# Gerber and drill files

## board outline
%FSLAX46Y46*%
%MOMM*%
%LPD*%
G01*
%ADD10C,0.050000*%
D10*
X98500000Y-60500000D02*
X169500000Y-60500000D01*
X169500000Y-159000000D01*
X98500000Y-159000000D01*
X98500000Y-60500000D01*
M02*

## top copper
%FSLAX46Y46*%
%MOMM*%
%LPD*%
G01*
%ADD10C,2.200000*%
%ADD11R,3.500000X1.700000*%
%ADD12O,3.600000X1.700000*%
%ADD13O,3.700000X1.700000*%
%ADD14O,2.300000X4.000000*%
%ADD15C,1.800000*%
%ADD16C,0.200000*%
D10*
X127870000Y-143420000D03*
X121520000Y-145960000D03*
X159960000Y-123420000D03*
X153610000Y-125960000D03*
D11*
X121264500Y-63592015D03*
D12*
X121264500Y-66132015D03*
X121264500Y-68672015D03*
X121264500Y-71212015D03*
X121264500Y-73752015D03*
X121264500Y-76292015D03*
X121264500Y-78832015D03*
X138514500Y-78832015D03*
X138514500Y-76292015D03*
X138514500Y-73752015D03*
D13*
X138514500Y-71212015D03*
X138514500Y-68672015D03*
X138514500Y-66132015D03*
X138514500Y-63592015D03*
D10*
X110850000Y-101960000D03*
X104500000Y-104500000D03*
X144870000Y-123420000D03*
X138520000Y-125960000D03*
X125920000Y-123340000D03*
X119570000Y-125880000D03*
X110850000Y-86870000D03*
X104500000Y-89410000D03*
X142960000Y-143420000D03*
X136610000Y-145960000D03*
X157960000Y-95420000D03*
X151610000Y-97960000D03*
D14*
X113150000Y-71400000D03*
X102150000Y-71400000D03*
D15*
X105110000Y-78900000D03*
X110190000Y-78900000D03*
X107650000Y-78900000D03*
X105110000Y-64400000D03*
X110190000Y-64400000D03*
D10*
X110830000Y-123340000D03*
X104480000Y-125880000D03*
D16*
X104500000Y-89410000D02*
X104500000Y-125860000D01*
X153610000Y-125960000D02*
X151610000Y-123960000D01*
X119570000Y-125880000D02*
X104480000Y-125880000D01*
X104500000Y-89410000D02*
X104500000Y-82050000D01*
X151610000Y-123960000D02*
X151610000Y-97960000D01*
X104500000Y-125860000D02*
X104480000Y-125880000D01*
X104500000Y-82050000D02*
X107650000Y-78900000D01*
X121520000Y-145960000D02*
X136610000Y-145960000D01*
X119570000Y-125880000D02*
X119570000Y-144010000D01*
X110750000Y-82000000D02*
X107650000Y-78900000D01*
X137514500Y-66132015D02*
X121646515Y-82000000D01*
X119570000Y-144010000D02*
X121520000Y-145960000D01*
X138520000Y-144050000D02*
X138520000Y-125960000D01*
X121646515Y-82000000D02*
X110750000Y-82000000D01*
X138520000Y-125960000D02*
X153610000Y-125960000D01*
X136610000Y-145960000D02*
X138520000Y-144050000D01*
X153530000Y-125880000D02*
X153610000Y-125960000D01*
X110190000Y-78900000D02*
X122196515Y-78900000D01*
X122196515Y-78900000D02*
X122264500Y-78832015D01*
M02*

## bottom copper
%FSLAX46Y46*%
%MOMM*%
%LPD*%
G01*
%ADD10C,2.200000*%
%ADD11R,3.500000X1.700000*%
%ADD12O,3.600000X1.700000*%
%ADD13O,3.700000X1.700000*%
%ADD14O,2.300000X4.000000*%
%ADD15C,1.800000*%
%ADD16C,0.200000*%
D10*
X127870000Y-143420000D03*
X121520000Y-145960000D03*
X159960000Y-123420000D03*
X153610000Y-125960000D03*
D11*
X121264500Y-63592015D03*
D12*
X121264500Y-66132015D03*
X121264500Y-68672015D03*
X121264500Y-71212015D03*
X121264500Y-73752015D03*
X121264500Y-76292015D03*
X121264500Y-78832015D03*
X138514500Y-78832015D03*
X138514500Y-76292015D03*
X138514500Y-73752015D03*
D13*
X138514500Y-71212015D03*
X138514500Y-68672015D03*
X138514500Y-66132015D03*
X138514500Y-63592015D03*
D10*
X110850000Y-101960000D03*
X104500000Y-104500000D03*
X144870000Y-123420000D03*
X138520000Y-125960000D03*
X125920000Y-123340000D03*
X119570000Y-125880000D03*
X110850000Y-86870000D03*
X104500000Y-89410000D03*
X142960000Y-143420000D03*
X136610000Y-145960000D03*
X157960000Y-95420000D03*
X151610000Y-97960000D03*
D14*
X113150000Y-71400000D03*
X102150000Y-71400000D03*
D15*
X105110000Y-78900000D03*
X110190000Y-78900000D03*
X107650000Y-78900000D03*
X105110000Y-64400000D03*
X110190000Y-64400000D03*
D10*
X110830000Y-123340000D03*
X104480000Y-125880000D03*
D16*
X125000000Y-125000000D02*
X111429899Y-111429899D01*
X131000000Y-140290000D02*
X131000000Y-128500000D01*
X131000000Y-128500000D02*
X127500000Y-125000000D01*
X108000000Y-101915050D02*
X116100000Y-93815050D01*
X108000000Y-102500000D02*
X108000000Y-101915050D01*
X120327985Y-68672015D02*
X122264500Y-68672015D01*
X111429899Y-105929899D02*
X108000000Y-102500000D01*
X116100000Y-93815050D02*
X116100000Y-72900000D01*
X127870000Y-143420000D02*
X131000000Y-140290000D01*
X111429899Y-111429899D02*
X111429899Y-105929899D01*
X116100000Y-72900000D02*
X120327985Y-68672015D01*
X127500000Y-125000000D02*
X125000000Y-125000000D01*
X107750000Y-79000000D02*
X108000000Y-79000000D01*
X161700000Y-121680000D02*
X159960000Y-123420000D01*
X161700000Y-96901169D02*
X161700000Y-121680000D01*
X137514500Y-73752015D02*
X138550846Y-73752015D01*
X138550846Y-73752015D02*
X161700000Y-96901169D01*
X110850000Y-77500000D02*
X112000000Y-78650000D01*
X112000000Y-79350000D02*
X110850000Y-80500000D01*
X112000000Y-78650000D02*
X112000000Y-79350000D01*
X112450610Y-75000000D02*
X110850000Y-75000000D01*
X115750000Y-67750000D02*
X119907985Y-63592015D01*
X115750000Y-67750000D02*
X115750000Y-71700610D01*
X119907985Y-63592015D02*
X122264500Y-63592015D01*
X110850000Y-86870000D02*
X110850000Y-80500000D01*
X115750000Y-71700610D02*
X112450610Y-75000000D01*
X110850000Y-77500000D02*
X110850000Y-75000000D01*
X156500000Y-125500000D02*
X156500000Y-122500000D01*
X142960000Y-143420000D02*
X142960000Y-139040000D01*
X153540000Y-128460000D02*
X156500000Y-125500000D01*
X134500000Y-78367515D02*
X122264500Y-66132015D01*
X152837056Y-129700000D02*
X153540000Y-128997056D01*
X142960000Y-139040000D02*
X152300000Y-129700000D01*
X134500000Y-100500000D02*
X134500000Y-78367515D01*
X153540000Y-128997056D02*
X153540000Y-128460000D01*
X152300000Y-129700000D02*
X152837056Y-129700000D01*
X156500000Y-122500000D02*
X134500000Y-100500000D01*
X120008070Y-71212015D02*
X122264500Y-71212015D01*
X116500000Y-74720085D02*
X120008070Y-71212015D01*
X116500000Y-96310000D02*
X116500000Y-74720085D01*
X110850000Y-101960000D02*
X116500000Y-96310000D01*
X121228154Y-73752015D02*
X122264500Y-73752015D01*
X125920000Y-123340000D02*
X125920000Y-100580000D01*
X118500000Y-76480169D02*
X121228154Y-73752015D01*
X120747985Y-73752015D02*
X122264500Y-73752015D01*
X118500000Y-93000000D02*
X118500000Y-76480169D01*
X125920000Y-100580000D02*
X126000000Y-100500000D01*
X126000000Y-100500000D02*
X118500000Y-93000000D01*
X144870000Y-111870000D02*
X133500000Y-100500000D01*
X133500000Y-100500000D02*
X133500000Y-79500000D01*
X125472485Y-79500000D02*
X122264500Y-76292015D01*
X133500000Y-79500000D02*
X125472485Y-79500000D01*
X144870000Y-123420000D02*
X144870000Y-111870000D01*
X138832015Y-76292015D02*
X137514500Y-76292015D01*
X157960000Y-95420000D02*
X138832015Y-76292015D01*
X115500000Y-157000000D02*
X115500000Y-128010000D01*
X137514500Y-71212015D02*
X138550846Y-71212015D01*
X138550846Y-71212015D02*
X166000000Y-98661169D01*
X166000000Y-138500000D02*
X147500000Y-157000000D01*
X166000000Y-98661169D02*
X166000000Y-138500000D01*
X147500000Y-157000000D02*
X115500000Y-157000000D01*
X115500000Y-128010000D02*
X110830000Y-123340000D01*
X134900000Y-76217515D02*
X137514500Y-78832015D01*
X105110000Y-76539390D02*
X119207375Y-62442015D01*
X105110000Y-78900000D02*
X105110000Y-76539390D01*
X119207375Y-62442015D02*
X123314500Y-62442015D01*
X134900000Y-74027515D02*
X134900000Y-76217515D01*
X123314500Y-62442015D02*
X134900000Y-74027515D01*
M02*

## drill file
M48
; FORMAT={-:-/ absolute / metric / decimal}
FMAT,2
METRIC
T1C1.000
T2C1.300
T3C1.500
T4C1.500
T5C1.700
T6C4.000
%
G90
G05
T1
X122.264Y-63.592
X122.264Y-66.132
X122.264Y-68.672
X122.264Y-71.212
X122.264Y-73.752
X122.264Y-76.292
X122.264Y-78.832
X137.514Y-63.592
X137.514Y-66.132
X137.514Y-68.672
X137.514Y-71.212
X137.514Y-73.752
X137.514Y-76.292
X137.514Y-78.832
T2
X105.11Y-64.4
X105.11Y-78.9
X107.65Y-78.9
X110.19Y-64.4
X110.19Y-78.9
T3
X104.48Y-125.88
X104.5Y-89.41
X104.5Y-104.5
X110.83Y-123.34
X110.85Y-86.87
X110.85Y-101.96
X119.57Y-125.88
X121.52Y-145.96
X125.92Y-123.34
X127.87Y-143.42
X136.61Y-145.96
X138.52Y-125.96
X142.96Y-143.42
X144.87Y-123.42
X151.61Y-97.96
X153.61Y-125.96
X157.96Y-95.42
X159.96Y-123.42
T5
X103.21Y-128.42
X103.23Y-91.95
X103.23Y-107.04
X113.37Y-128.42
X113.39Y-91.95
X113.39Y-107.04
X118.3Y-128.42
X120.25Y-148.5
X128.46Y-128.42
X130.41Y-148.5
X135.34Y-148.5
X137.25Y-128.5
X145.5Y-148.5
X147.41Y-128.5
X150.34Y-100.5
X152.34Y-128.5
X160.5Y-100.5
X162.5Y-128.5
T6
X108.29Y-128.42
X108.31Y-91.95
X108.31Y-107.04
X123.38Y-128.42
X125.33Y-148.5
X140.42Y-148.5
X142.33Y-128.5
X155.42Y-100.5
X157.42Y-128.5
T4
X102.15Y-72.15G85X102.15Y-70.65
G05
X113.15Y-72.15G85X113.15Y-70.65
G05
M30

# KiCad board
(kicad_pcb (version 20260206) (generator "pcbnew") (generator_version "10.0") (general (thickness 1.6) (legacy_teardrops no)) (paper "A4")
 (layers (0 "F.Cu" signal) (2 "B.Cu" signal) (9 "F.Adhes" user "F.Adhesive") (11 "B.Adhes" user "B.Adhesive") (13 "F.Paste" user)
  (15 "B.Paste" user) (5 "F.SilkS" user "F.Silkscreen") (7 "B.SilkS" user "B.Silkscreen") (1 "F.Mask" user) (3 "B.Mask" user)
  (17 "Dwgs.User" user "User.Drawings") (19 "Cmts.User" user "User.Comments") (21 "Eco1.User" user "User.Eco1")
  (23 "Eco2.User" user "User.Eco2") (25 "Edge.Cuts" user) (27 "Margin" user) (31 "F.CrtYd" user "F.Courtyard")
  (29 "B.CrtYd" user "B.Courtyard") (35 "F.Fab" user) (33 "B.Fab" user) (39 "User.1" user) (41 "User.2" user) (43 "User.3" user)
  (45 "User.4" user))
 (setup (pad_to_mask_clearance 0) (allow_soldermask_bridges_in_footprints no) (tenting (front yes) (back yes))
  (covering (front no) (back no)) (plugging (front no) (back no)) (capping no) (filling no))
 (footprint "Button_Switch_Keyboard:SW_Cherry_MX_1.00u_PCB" (layer "F.Cu") (at 127.87 143.42)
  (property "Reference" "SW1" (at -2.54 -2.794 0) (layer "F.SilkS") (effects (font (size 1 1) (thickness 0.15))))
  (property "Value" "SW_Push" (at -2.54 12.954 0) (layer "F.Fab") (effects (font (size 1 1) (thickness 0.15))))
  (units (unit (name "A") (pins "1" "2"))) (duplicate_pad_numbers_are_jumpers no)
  (pad "" np_thru_hole circle (at -7.62 5.08) (size 1.7 1.7) (drill 1.7) (layers "*.Cu" "*.Mask"))
  (pad "" np_thru_hole circle (at -2.54 5.08) (size 4 4) (drill 4) (layers "*.Cu" "*.Mask"))
  (pad "" np_thru_hole circle (at 2.54 5.08) (size 1.7 1.7) (drill 1.7) (layers "*.Cu" "*.Mask"))
  (pad "1" thru_hole circle (at 0 0) (size 2.2 2.2) (drill 1.5) (layers "*.Cu" "*.Mask") (remove_unused_layers no)
   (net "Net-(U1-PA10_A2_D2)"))
  (pad "2" thru_hole circle (at -6.35 2.54) (size 2.2 2.2) (drill 1.5) (layers "*.Cu" "*.Mask") (remove_unused_layers no) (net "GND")))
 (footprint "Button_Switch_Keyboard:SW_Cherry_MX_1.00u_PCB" (layer "F.Cu") (at 159.96 123.42)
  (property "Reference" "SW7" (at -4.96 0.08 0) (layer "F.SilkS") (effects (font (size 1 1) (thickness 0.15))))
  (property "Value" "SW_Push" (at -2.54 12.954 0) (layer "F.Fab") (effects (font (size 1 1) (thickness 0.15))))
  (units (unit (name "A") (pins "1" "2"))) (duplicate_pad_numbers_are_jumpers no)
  (pad "" np_thru_hole circle (at -7.62 5.08) (size 1.7 1.7) (drill 1.7) (layers "*.Cu" "*.Mask"))
  (pad "" np_thru_hole circle (at -2.54 5.08) (size 4 4) (drill 4) (layers "*.Cu" "*.Mask"))
  (pad "" np_thru_hole circle (at 2.54 5.08) (size 1.7 1.7) (drill 1.7) (layers "*.Cu" "*.Mask"))
  (pad "1" thru_hole circle (at 0 0) (size 2.2 2.2) (drill 1.5) (layers "*.Cu" "*.Mask") (remove_unused_layers no)
   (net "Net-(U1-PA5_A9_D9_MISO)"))
  (pad "2" thru_hole circle (at -6.35 2.54) (size 2.2 2.2) (drill 1.5) (layers "*.Cu" "*.Mask") (remove_unused_layers no) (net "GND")))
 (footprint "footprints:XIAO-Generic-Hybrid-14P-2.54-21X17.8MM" (layer "F.Cu") (at 129.8895 71.212015)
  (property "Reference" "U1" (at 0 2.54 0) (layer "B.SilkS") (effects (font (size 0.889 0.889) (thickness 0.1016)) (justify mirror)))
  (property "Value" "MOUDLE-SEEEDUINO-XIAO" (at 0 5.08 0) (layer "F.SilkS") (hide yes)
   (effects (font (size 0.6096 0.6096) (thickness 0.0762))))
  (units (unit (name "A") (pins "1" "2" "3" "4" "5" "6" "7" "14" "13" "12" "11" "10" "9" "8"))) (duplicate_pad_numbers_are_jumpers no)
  (pad "1" thru_hole rect (at -7.625 -7.62) (size 3.5 1.7) (drill 1 (offset -1 0)) (layers "*.Cu" "*.Mask") (remove_unused_layers no)
   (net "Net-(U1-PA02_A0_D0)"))
  (pad "2" thru_hole oval (at -7.625 -5.08) (size 3.6 1.7) (drill 1 (offset -1 0)) (layers "*.Cu" "*.Mask") (remove_unused_layers no)
   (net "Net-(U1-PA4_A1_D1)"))
  (pad "3" thru_hole oval (at -7.625 -2.54) (size 3.6 1.7) (drill 1 (offset -1 0)) (layers "*.Cu" "*.Mask") (remove_unused_layers no)
   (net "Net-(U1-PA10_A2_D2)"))
  (pad "4" thru_hole oval (at -7.625 0) (size 3.6 1.7) (drill 1 (offset -1 0)) (layers "*.Cu" "*.Mask") (remove_unused_layers no)
   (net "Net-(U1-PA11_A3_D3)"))
  (pad "5" thru_hole oval (at -7.625 2.54) (size 3.6 1.7) (drill 1 (offset -1 0)) (layers "*.Cu" "*.Mask") (remove_unused_layers no)
   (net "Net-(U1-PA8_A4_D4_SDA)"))
  (pad "6" thru_hole oval (at -7.625 5.08 180) (size 3.6 1.7) (drill 1 (offset 1 0)) (layers "*.Cu" "*.Mask") (remove_unused_layers no)
   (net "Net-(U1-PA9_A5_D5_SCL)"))
  (pad "7" thru_hole oval (at -7.625 7.62) (size 3.6 1.7) (drill 1 (offset -1 0)) (layers "*.Cu" "*.Mask") (remove_unused_layers no)
   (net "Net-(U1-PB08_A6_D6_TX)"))
  (pad "8" thru_hole oval (at 7.625 7.62) (size 3.6 1.7) (drill 1 (offset 1 0)) (layers "*.Cu" "*.Mask") (remove_unused_layers no)
   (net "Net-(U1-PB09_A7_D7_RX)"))
  (pad "9" thru_hole oval (at 7.625 5.08) (size 3.6 1.7) (drill 1 (offset 1 0)) (layers "*.Cu" "*.Mask") (remove_unused_layers no)
   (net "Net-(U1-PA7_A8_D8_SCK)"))
  (pad "10" thru_hole oval (at 7.625 2.54) (size 3.6 1.7) (drill 1 (offset 1 0)) (layers "*.Cu" "*.Mask") (remove_unused_layers no)
   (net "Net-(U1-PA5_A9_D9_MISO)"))
  (pad "11" thru_hole oval (at 7.625 0) (size 3.7 1.7) (drill 1 (offset 1 0)) (layers "*.Cu" "*.Mask") (remove_unused_layers no)
   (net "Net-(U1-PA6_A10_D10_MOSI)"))
  (pad "12" thru_hole oval (at 7.625 -2.54) (size 3.7 1.7) (drill 1 (offset 1 0)) (layers "*.Cu" "*.Mask") (remove_unused_layers no)
   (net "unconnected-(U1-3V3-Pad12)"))
  (pad "13" thru_hole oval (at 7.625 -5.08) (size 3.7 1.7) (drill 1 (offset 1 0)) (layers "*.Cu" "*.Mask") (remove_unused_layers no)
   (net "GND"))
  (pad "14" thru_hole oval (at 7.625 -7.62) (size 3.7 1.7) (drill 1 (offset 1 0)) (layers "*.Cu" "*.Mask") (remove_unused_layers no)
   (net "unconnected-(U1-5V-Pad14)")))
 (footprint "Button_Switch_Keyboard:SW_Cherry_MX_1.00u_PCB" (layer "F.Cu") (at 110.85 101.96)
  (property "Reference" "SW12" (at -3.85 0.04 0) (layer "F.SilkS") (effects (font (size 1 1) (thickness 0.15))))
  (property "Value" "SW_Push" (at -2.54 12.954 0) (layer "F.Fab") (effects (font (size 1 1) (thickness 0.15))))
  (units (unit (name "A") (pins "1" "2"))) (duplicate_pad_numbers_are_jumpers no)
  (pad "" np_thru_hole circle (at -7.62 5.08) (size 1.7 1.7) (drill 1.7) (layers "*.Cu" "*.Mask"))
  (pad "" np_thru_hole circle (at -2.54 5.08) (size 4 4) (drill 4) (layers "*.Cu" "*.Mask"))
  (pad "" np_thru_hole circle (at 2.54 5.08) (size 1.7 1.7) (drill 1.7) (layers "*.Cu" "*.Mask"))
  (pad "1" thru_hole circle (at 0 0) (size 2.2 2.2) (drill 1.5) (layers "*.Cu" "*.Mask") (remove_unused_layers no)
   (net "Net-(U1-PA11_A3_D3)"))
  (pad "2" thru_hole circle (at -6.35 2.54) (size 2.2 2.2) (drill 1.5) (layers "*.Cu" "*.Mask") (remove_unused_layers no) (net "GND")))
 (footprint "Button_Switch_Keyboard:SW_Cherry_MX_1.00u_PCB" (layer "F.Cu") (at 144.87 123.42)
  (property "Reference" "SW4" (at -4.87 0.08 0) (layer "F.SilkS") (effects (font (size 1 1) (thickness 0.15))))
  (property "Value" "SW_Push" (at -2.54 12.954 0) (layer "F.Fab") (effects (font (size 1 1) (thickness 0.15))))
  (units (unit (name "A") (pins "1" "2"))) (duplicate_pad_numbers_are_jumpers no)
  (pad "" np_thru_hole circle (at -7.62 5.08) (size 1.7 1.7) (drill 1.7) (layers "*.Cu" "*.Mask"))
  (pad "" np_thru_hole circle (at -2.54 5.08) (size 4 4) (drill 4) (layers "*.Cu" "*.Mask"))
  (pad "" np_thru_hole circle (at 2.54 5.08) (size 1.7 1.7) (drill 1.7) (layers "*.Cu" "*.Mask"))
  (pad "1" thru_hole circle (at 0 0) (size 2.2 2.2) (drill 1.5) (layers "*.Cu" "*.Mask") (remove_unused_layers no)
   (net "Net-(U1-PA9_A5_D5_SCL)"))
  (pad "2" thru_hole circle (at -6.35 2.54) (size 2.2 2.2) (drill 1.5) (layers "*.Cu" "*.Mask") (remove_unused_layers no) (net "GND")))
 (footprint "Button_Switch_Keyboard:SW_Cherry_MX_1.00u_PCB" (layer "F.Cu") (at 125.92 123.34)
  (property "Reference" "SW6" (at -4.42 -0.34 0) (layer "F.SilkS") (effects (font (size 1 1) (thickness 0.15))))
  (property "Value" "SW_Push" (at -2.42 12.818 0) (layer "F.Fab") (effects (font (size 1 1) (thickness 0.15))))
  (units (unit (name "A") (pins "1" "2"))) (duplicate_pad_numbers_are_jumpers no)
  (pad "" np_thru_hole circle (at -7.62 5.08) (size 1.7 1.7) (drill 1.7) (layers "*.Cu" "*.Mask"))
  (pad "" np_thru_hole circle (at -2.54 5.08) (size 4 4) (drill 4) (layers "*.Cu" "*.Mask"))
  (pad "" np_thru_hole circle (at 2.54 5.08) (size 1.7 1.7) (drill 1.7) (layers "*.Cu" "*.Mask"))
  (pad "1" thru_hole circle (at 0 0) (size 2.2 2.2) (drill 1.5) (layers "*.Cu" "*.Mask") (remove_unused_layers no)
   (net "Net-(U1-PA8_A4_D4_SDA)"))
  (pad "2" thru_hole circle (at -6.35 2.54) (size 2.2 2.2) (drill 1.5) (layers "*.Cu" "*.Mask") (remove_unused_layers no) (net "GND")))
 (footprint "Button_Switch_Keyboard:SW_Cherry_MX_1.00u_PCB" (layer "F.Cu") (at 110.85 86.87)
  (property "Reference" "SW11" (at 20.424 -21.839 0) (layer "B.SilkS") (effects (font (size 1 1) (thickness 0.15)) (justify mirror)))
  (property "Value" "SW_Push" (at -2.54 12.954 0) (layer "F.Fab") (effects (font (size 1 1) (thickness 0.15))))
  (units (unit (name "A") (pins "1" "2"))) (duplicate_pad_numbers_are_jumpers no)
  (pad "" np_thru_hole circle (at -7.62 5.08) (size 1.7 1.7) (drill 1.7) (layers "*.Cu" "*.Mask"))
  (pad "" np_thru_hole circle (at -2.54 5.08) (size 4 4) (drill 4) (layers "*.Cu" "*.Mask"))
  (pad "" np_thru_hole circle (at 2.54 5.08) (size 1.7 1.7) (drill 1.7) (layers "*.Cu" "*.Mask"))
  (pad "1" thru_hole circle (at 0 0) (size 2.2 2.2) (drill 1.5) (layers "*.Cu" "*.Mask") (remove_unused_layers no)
   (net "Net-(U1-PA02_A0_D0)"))
  (pad "2" thru_hole circle (at -6.35 2.54) (size 2.2 2.2) (drill 1.5) (layers "*.Cu" "*.Mask") (remove_unused_layers no) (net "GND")))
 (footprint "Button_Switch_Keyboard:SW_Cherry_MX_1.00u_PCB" (layer "F.Cu") (at 142.96 143.42)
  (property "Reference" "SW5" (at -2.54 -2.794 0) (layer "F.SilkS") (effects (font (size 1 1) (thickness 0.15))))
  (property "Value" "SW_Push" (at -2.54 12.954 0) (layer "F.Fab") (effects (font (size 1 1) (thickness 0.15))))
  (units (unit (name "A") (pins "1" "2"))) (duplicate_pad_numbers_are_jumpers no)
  (pad "" np_thru_hole circle (at -7.62 5.08) (size 1.7 1.7) (drill 1.7) (layers "*.Cu" "*.Mask"))
  (pad "" np_thru_hole circle (at -2.54 5.08) (size 4 4) (drill 4) (layers "*.Cu" "*.Mask"))
  (pad "" np_thru_hole circle (at 2.54 5.08) (size 1.7 1.7) (drill 1.7) (layers "*.Cu" "*.Mask"))
  (pad "1" thru_hole circle (at 0 0) (size 2.2 2.2) (drill 1.5) (layers "*.Cu" "*.Mask") (remove_unused_layers no)
   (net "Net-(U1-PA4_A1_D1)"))
  (pad "2" thru_hole circle (at -6.35 2.54) (size 2.2 2.2) (drill 1.5) (layers "*.Cu" "*.Mask") (remove_unused_layers no) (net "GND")))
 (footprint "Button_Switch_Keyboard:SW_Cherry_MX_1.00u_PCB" (layer "F.Cu") (at 157.96 95.42)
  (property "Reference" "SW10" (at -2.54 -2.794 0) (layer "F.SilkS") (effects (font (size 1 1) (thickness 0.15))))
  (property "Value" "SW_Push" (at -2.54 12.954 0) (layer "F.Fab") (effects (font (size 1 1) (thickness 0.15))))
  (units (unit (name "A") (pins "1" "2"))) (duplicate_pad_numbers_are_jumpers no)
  (pad "" np_thru_hole circle (at -7.62 5.08) (size 1.7 1.7) (drill 1.7) (layers "*.Cu" "*.Mask"))
  (pad "" np_thru_hole circle (at -2.54 5.08) (size 4 4) (drill 4) (layers "*.Cu" "*.Mask"))
  (pad "" np_thru_hole circle (at 2.54 5.08) (size 1.7 1.7) (drill 1.7) (layers "*.Cu" "*.Mask"))
  (pad "1" thru_hole circle (at 0 0) (size 2.2 2.2) (drill 1.5) (layers "*.Cu" "*.Mask") (remove_unused_layers no)
   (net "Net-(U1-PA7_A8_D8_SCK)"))
  (pad "2" thru_hole circle (at -6.35 2.54) (size 2.2 2.2) (drill 1.5) (layers "*.Cu" "*.Mask") (remove_unused_layers no) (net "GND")))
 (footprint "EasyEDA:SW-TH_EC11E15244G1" (layer "F.Cu") (at 107.65 71.65)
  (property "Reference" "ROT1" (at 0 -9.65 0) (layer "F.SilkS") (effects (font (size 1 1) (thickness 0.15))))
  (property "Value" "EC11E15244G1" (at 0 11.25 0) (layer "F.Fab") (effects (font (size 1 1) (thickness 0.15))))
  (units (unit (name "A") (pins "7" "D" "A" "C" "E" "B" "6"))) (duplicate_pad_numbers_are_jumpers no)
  (pad "6" thru_hole oval (at 5.5 -0.25 90) (size 4 2.3) (drill oval 2.999994 1.500022) (layers "*.Cu" "*.Mask") (remove_unused_layers no)
   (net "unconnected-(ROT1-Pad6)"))
  (pad "7" thru_hole oval (at -5.5 -0.25 90) (size 4 2.3) (drill oval 2.999994 1.500022) (layers "*.Cu" "*.Mask") (remove_unused_layers no)
   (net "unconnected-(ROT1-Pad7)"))
  (pad "A" thru_hole circle (at -2.54 7.25) (size 1.8 1.8) (drill 1.300022) (layers "*.Cu" "*.Mask") (remove_unused_layers no)
   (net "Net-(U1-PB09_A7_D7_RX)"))
  (pad "B" thru_hole circle (at 2.54 7.25) (size 1.8 1.8) (drill 1.300022) (layers "*.Cu" "*.Mask") (remove_unused_layers no)
   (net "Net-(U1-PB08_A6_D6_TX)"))
  (pad "C" thru_hole circle (at 0 7.25) (size 1.8 1.8) (drill 1.300022) (layers "*.Cu" "*.Mask") (remove_unused_layers no) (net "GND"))
  (pad "D" thru_hole circle (at -2.54 -7.25) (size 1.8 1.8) (drill 1.300022) (layers "*.Cu" "*.Mask") (remove_unused_layers no)
   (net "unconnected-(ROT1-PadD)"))
  (pad "E" thru_hole circle (at 2.54 -7.25) (size 1.8 1.8) (drill 1.300022) (layers "*.Cu" "*.Mask") (remove_unused_layers no)
   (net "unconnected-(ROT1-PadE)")))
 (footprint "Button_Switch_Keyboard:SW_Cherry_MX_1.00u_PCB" (layer "F.Cu") (at 110.83 123.34)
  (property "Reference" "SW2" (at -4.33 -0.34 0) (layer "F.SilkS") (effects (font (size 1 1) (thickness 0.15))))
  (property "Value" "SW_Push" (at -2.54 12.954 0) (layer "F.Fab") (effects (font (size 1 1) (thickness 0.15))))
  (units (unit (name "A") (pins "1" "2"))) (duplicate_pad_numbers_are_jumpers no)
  (pad "" np_thru_hole circle (at -7.62 5.08) (size 1.7 1.7) (drill 1.7) (layers "*.Cu" "*.Mask"))
  (pad "" np_thru_hole circle (at -2.54 5.08) (size 4 4) (drill 4) (layers "*.Cu" "*.Mask"))
  (pad "" np_thru_hole circle (at 2.54 5.08) (size 1.7 1.7) (drill 1.7) (layers "*.Cu" "*.Mask"))
  (pad "1" thru_hole circle (at 0 0) (size 2.2 2.2) (drill 1.5) (layers "*.Cu" "*.Mask") (remove_unused_layers no)
   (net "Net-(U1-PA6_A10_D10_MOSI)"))
  (pad "2" thru_hole circle (at -6.35 2.54) (size 2.2 2.2) (drill 1.5) (layers "*.Cu" "*.Mask") (remove_unused_layers no) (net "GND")))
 (gr_rect (start 98.5 60.5) (end 169.5 159) (stroke (width 0.05) (type default)) (fill no) (layer "Edge.Cuts"))
 (segment (start 125 125) (end 111.429899 111.429899) (width 0.2) (layer "B.Cu") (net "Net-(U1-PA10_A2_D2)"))
 (segment (start 131 140.29) (end 131 128.5) (width 0.2) (layer "B.Cu") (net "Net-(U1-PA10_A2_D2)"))
 (segment (start 131 128.5) (end 127.5 125) (width 0.2) (layer "B.Cu") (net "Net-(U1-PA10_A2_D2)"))
 (segment (start 108 101.91505) (end 116.1 93.81505) (width 0.2) (layer "B.Cu") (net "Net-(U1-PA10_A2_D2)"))
 (segment (start 108 102.5) (end 108 101.91505) (width 0.2) (layer "B.Cu") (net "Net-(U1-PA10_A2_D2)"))
 (segment (start 120.327985 68.672015) (end 122.2645 68.672015) (width 0.2) (layer "B.Cu") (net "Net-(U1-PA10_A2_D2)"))
 (segment (start 111.429899 105.929899) (end 108 102.5) (width 0.2) (layer "B.Cu") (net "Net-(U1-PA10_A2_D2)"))
 (segment (start 116.1 93.81505) (end 116.1 72.9) (width 0.2) (layer "B.Cu") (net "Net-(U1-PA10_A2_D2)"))
 (segment (start 127.87 143.42) (end 131 140.29) (width 0.2) (layer "B.Cu") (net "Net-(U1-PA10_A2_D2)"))
 (segment (start 111.429899 111.429899) (end 111.429899 105.929899) (width 0.2) (layer "B.Cu") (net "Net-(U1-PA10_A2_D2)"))
 (segment (start 116.1 72.9) (end 120.327985 68.672015) (width 0.2) (layer "B.Cu") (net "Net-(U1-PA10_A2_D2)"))
 (segment (start 127.5 125) (end 125 125) (width 0.2) (layer "B.Cu") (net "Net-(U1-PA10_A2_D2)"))
 (segment (start 104.5 89.41) (end 104.5 125.86) (width 0.2) (layer "F.Cu") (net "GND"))
 (segment (start 153.61 125.96) (end 151.61 123.96) (width 0.2) (layer "F.Cu") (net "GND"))
 (segment (start 119.57 125.88) (end 104.48 125.88) (width 0.2) (layer "F.Cu") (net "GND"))
 (segment (start 104.5 89.41) (end 104.5 82.05) (width 0.2) (layer "F.Cu") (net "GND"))
 (segment (start 151.61 123.96) (end 151.61 97.96) (width 0.2) (layer "F.Cu") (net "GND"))
 (segment (start 104.5 125.86) (end 104.48 125.88) (width 0.2) (layer "F.Cu") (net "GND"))
 (segment (start 104.5 82.05) (end 107.65 78.9) (width 0.2) (layer "F.Cu") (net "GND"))
 (segment (start 121.52 145.96) (end 136.61 145.96) (width 0.2) (layer "F.Cu") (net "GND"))
 (segment (start 119.57 125.88) (end 119.57 144.01) (width 0.2) (layer "F.Cu") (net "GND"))
 (segment (start 110.75 82) (end 107.65 78.9) (width 0.2) (layer "F.Cu") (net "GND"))
 (segment (start 137.5145 66.132015) (end 121.646515 82) (width 0.2) (layer "F.Cu") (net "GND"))
 (segment (start 119.57 144.01) (end 121.52 145.96) (width 0.2) (layer "F.Cu") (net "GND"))
 (segment (start 138.52 144.05) (end 138.52 125.96) (width 0.2) (layer "F.Cu") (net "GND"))
 (segment (start 121.646515 82) (end 110.75 82) (width 0.2) (layer "F.Cu") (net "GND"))
 (segment (start 138.52 125.96) (end 153.61 125.96) (width 0.2) (layer "F.Cu") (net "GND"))
 (segment (start 136.61 145.96) (end 138.52 144.05) (width 0.2) (layer "F.Cu") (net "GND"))
 (segment (start 153.53 125.88) (end 153.61 125.96) (width 0.2) (layer "F.Cu") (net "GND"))
 (segment (start 107.75 79) (end 108 79) (width 0.2) (layer "B.Cu") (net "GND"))
 (segment (start 161.7 121.68) (end 159.96 123.42) (width 0.2) (layer "B.Cu") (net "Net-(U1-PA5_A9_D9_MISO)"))
 (segment (start 161.7 96.901169) (end 161.7 121.68) (width 0.2) (layer "B.Cu") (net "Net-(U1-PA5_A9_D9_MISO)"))
 (segment (start 137.5145 73.752015) (end 138.550846 73.752015) (width 0.2) (layer "B.Cu") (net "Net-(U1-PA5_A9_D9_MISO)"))
 (segment (start 138.550846 73.752015) (end 161.7 96.901169) (width 0.2) (layer "B.Cu") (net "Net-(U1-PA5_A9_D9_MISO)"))
 (segment (start 110.85 77.5) (end 112 78.65) (width 0.2) (layer "B.Cu") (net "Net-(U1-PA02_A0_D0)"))
 (segment (start 112 79.35) (end 110.85 80.5) (width 0.2) (layer "B.Cu") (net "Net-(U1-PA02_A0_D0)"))
 (segment (start 112 78.65) (end 112 79.35) (width 0.2) (layer "B.Cu") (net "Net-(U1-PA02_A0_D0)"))
 (segment (start 112.45061 75) (end 110.85 75) (width 0.2) (layer "B.Cu") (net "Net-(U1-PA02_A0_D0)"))
 (segment (start 115.75 67.75) (end 119.907985 63.592015) (width 0.2) (layer "B.Cu") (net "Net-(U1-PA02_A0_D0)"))
 (segment (start 115.75 67.75) (end 115.75 71.70061) (width 0.2) (layer "B.Cu") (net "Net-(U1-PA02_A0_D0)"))
 (segment (start 119.907985 63.592015) (end 122.2645 63.592015) (width 0.2) (layer "B.Cu") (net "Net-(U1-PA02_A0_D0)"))
 (segment (start 110.85 86.87) (end 110.85 80.5) (width 0.2) (layer "B.Cu") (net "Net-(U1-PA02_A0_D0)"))
 (segment (start 115.75 71.70061) (end 112.45061 75) (width 0.2) (layer "B.Cu") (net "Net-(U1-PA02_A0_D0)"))
 (segment (start 110.85 77.5) (end 110.85 75) (width 0.2) (layer "B.Cu") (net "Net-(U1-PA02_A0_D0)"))
 (segment (start 156.5 125.5) (end 156.5 122.5) (width 0.2) (layer "B.Cu") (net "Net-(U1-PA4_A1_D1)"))
 (segment (start 142.96 143.42) (end 142.96 139.04) (width 0.2) (layer "B.Cu") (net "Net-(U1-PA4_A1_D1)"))
 (segment (start 153.54 128.46) (end 156.5 125.5) (width 0.2) (layer "B.Cu") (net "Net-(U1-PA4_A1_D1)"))
 (segment (start 134.5 78.367515) (end 122.2645 66.132015) (width 0.2) (layer "B.Cu") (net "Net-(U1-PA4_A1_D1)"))
 (segment (start 152.837056 129.7) (end 153.54 128.997056) (width 0.2) (layer "B.Cu") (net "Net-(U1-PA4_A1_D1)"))
 (segment (start 142.96 139.04) (end 152.3 129.7) (width 0.2) (layer "B.Cu") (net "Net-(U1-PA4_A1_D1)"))
 (segment (start 134.5 100.5) (end 134.5 78.367515) (width 0.2) (layer "B.Cu") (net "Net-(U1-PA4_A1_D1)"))
 (segment (start 153.54 128.997056) (end 153.54 128.46) (width 0.2) (layer "B.Cu") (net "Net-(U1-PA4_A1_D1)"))
 (segment (start 152.3 129.7) (end 152.837056 129.7) (width 0.2) (layer "B.Cu") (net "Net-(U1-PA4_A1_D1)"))
 (segment (start 156.5 122.5) (end 134.5 100.5) (width 0.2) (layer "B.Cu") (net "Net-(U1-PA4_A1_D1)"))
 (segment (start 120.00807 71.212015) (end 122.2645 71.212015) (width 0.2) (layer "B.Cu") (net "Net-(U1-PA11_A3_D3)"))
 (segment (start 116.5 74.720085) (end 120.00807 71.212015) (width 0.2) (layer "B.Cu") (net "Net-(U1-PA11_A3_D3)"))
 (segment (start 116.5 96.31) (end 116.5 74.720085) (width 0.2) (layer "B.Cu") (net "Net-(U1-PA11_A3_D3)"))
 (segment (start 110.85 101.96) (end 116.5 96.31) (width 0.2) (layer "B.Cu") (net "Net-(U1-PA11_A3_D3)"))
 (segment (start 121.228154 73.752015) (end 122.2645 73.752015) (width 0.2) (layer "B.Cu") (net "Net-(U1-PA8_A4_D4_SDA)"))
 (segment (start 125.92 123.34) (end 125.92 100.58) (width 0.2) (layer "B.Cu") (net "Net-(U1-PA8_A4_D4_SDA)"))
 (segment (start 118.5 76.480169) (end 121.228154 73.752015) (width 0.2) (layer "B.Cu") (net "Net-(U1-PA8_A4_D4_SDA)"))
 (segment (start 120.747985 73.752015) (end 122.2645 73.752015) (width 0.2) (layer "B.Cu") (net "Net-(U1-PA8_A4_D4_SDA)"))
 (segment (start 118.5 93) (end 118.5 76.480169) (width 0.2) (layer "B.Cu") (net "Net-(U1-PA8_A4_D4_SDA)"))
 (segment (start 125.92 100.58) (end 126 100.5) (width 0.2) (layer "B.Cu") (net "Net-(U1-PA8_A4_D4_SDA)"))
 (segment (start 126 100.5) (end 118.5 93) (width 0.2) (layer "B.Cu") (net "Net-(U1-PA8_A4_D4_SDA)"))
 (segment (start 144.87 111.87) (end 133.5 100.5) (width 0.2) (layer "B.Cu") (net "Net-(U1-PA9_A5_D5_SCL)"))
 (segment (start 133.5 100.5) (end 133.5 79.5) (width 0.2) (layer "B.Cu") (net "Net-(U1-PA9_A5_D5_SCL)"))
 (segment (start 125.472485 79.5) (end 122.2645 76.292015) (width 0.2) (layer "B.Cu") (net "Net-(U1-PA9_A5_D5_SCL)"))
 (segment (start 133.5 79.5) (end 125.472485 79.5) (width 0.2) (layer "B.Cu") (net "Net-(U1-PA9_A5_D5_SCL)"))
 (segment (start 144.87 123.42) (end 144.87 111.87) (width 0.2) (layer "B.Cu") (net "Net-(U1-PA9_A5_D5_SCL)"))
 (segment (start 138.832015 76.292015) (end 137.5145 76.292015) (width 0.2) (layer "B.Cu") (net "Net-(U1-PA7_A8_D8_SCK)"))
 (segment (start 157.96 95.42) (end 138.832015 76.292015) (width 0.2) (layer "B.Cu") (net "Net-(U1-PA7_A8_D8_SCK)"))
 (segment (start 115.5 157) (end 115.5 128.01) (width 0.2) (layer "B.Cu") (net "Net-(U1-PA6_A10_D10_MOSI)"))
 (segment (start 137.5145 71.212015) (end 138.550846 71.212015) (width 0.2) (layer "B.Cu") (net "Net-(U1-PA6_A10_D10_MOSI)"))
 (segment (start 138.550846 71.212015) (end 166 98.661169) (width 0.2) (layer "B.Cu") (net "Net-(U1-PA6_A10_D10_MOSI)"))
 (segment (start 166 138.5) (end 147.5 157) (width 0.2) (layer "B.Cu") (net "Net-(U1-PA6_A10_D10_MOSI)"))
 (segment (start 166 98.661169) (end 166 138.5) (width 0.2) (layer "B.Cu") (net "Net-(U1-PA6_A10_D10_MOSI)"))
 (segment (start 147.5 157) (end 115.5 157) (width 0.2) (layer "B.Cu") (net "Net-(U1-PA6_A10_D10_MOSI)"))
 (segment (start 115.5 128.01) (end 110.83 123.34) (width 0.2) (layer "B.Cu") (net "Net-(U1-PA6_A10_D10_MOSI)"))
 (segment (start 134.9 76.217515) (end 137.5145 78.832015) (width 0.2) (layer "B.Cu") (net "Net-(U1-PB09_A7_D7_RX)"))
 (segment (start 105.11 76.53939) (end 119.207375 62.442015) (width 0.2) (layer "B.Cu") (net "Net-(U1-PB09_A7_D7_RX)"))
 (segment (start 105.11 78.9) (end 105.11 76.53939) (width 0.2) (layer "B.Cu") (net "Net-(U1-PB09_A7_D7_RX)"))
 (segment (start 119.207375 62.442015) (end 123.3145 62.442015) (width 0.2) (layer "B.Cu") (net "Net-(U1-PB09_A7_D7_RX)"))
 (segment (start 134.9 74.027515) (end 134.9 76.217515) (width 0.2) (layer "B.Cu") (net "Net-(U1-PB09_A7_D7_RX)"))
 (segment (start 123.3145 62.442015) (end 134.9 74.027515) (width 0.2) (layer "B.Cu") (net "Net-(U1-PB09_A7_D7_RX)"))
 (segment (start 110.19 78.9) (end 122.196515 78.9) (width 0.2) (layer "F.Cu") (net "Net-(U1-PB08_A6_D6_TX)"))
 (segment (start 122.196515 78.9) (end 122.2645 78.832015) (width 0.2) (layer "F.Cu") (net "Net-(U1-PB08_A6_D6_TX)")))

